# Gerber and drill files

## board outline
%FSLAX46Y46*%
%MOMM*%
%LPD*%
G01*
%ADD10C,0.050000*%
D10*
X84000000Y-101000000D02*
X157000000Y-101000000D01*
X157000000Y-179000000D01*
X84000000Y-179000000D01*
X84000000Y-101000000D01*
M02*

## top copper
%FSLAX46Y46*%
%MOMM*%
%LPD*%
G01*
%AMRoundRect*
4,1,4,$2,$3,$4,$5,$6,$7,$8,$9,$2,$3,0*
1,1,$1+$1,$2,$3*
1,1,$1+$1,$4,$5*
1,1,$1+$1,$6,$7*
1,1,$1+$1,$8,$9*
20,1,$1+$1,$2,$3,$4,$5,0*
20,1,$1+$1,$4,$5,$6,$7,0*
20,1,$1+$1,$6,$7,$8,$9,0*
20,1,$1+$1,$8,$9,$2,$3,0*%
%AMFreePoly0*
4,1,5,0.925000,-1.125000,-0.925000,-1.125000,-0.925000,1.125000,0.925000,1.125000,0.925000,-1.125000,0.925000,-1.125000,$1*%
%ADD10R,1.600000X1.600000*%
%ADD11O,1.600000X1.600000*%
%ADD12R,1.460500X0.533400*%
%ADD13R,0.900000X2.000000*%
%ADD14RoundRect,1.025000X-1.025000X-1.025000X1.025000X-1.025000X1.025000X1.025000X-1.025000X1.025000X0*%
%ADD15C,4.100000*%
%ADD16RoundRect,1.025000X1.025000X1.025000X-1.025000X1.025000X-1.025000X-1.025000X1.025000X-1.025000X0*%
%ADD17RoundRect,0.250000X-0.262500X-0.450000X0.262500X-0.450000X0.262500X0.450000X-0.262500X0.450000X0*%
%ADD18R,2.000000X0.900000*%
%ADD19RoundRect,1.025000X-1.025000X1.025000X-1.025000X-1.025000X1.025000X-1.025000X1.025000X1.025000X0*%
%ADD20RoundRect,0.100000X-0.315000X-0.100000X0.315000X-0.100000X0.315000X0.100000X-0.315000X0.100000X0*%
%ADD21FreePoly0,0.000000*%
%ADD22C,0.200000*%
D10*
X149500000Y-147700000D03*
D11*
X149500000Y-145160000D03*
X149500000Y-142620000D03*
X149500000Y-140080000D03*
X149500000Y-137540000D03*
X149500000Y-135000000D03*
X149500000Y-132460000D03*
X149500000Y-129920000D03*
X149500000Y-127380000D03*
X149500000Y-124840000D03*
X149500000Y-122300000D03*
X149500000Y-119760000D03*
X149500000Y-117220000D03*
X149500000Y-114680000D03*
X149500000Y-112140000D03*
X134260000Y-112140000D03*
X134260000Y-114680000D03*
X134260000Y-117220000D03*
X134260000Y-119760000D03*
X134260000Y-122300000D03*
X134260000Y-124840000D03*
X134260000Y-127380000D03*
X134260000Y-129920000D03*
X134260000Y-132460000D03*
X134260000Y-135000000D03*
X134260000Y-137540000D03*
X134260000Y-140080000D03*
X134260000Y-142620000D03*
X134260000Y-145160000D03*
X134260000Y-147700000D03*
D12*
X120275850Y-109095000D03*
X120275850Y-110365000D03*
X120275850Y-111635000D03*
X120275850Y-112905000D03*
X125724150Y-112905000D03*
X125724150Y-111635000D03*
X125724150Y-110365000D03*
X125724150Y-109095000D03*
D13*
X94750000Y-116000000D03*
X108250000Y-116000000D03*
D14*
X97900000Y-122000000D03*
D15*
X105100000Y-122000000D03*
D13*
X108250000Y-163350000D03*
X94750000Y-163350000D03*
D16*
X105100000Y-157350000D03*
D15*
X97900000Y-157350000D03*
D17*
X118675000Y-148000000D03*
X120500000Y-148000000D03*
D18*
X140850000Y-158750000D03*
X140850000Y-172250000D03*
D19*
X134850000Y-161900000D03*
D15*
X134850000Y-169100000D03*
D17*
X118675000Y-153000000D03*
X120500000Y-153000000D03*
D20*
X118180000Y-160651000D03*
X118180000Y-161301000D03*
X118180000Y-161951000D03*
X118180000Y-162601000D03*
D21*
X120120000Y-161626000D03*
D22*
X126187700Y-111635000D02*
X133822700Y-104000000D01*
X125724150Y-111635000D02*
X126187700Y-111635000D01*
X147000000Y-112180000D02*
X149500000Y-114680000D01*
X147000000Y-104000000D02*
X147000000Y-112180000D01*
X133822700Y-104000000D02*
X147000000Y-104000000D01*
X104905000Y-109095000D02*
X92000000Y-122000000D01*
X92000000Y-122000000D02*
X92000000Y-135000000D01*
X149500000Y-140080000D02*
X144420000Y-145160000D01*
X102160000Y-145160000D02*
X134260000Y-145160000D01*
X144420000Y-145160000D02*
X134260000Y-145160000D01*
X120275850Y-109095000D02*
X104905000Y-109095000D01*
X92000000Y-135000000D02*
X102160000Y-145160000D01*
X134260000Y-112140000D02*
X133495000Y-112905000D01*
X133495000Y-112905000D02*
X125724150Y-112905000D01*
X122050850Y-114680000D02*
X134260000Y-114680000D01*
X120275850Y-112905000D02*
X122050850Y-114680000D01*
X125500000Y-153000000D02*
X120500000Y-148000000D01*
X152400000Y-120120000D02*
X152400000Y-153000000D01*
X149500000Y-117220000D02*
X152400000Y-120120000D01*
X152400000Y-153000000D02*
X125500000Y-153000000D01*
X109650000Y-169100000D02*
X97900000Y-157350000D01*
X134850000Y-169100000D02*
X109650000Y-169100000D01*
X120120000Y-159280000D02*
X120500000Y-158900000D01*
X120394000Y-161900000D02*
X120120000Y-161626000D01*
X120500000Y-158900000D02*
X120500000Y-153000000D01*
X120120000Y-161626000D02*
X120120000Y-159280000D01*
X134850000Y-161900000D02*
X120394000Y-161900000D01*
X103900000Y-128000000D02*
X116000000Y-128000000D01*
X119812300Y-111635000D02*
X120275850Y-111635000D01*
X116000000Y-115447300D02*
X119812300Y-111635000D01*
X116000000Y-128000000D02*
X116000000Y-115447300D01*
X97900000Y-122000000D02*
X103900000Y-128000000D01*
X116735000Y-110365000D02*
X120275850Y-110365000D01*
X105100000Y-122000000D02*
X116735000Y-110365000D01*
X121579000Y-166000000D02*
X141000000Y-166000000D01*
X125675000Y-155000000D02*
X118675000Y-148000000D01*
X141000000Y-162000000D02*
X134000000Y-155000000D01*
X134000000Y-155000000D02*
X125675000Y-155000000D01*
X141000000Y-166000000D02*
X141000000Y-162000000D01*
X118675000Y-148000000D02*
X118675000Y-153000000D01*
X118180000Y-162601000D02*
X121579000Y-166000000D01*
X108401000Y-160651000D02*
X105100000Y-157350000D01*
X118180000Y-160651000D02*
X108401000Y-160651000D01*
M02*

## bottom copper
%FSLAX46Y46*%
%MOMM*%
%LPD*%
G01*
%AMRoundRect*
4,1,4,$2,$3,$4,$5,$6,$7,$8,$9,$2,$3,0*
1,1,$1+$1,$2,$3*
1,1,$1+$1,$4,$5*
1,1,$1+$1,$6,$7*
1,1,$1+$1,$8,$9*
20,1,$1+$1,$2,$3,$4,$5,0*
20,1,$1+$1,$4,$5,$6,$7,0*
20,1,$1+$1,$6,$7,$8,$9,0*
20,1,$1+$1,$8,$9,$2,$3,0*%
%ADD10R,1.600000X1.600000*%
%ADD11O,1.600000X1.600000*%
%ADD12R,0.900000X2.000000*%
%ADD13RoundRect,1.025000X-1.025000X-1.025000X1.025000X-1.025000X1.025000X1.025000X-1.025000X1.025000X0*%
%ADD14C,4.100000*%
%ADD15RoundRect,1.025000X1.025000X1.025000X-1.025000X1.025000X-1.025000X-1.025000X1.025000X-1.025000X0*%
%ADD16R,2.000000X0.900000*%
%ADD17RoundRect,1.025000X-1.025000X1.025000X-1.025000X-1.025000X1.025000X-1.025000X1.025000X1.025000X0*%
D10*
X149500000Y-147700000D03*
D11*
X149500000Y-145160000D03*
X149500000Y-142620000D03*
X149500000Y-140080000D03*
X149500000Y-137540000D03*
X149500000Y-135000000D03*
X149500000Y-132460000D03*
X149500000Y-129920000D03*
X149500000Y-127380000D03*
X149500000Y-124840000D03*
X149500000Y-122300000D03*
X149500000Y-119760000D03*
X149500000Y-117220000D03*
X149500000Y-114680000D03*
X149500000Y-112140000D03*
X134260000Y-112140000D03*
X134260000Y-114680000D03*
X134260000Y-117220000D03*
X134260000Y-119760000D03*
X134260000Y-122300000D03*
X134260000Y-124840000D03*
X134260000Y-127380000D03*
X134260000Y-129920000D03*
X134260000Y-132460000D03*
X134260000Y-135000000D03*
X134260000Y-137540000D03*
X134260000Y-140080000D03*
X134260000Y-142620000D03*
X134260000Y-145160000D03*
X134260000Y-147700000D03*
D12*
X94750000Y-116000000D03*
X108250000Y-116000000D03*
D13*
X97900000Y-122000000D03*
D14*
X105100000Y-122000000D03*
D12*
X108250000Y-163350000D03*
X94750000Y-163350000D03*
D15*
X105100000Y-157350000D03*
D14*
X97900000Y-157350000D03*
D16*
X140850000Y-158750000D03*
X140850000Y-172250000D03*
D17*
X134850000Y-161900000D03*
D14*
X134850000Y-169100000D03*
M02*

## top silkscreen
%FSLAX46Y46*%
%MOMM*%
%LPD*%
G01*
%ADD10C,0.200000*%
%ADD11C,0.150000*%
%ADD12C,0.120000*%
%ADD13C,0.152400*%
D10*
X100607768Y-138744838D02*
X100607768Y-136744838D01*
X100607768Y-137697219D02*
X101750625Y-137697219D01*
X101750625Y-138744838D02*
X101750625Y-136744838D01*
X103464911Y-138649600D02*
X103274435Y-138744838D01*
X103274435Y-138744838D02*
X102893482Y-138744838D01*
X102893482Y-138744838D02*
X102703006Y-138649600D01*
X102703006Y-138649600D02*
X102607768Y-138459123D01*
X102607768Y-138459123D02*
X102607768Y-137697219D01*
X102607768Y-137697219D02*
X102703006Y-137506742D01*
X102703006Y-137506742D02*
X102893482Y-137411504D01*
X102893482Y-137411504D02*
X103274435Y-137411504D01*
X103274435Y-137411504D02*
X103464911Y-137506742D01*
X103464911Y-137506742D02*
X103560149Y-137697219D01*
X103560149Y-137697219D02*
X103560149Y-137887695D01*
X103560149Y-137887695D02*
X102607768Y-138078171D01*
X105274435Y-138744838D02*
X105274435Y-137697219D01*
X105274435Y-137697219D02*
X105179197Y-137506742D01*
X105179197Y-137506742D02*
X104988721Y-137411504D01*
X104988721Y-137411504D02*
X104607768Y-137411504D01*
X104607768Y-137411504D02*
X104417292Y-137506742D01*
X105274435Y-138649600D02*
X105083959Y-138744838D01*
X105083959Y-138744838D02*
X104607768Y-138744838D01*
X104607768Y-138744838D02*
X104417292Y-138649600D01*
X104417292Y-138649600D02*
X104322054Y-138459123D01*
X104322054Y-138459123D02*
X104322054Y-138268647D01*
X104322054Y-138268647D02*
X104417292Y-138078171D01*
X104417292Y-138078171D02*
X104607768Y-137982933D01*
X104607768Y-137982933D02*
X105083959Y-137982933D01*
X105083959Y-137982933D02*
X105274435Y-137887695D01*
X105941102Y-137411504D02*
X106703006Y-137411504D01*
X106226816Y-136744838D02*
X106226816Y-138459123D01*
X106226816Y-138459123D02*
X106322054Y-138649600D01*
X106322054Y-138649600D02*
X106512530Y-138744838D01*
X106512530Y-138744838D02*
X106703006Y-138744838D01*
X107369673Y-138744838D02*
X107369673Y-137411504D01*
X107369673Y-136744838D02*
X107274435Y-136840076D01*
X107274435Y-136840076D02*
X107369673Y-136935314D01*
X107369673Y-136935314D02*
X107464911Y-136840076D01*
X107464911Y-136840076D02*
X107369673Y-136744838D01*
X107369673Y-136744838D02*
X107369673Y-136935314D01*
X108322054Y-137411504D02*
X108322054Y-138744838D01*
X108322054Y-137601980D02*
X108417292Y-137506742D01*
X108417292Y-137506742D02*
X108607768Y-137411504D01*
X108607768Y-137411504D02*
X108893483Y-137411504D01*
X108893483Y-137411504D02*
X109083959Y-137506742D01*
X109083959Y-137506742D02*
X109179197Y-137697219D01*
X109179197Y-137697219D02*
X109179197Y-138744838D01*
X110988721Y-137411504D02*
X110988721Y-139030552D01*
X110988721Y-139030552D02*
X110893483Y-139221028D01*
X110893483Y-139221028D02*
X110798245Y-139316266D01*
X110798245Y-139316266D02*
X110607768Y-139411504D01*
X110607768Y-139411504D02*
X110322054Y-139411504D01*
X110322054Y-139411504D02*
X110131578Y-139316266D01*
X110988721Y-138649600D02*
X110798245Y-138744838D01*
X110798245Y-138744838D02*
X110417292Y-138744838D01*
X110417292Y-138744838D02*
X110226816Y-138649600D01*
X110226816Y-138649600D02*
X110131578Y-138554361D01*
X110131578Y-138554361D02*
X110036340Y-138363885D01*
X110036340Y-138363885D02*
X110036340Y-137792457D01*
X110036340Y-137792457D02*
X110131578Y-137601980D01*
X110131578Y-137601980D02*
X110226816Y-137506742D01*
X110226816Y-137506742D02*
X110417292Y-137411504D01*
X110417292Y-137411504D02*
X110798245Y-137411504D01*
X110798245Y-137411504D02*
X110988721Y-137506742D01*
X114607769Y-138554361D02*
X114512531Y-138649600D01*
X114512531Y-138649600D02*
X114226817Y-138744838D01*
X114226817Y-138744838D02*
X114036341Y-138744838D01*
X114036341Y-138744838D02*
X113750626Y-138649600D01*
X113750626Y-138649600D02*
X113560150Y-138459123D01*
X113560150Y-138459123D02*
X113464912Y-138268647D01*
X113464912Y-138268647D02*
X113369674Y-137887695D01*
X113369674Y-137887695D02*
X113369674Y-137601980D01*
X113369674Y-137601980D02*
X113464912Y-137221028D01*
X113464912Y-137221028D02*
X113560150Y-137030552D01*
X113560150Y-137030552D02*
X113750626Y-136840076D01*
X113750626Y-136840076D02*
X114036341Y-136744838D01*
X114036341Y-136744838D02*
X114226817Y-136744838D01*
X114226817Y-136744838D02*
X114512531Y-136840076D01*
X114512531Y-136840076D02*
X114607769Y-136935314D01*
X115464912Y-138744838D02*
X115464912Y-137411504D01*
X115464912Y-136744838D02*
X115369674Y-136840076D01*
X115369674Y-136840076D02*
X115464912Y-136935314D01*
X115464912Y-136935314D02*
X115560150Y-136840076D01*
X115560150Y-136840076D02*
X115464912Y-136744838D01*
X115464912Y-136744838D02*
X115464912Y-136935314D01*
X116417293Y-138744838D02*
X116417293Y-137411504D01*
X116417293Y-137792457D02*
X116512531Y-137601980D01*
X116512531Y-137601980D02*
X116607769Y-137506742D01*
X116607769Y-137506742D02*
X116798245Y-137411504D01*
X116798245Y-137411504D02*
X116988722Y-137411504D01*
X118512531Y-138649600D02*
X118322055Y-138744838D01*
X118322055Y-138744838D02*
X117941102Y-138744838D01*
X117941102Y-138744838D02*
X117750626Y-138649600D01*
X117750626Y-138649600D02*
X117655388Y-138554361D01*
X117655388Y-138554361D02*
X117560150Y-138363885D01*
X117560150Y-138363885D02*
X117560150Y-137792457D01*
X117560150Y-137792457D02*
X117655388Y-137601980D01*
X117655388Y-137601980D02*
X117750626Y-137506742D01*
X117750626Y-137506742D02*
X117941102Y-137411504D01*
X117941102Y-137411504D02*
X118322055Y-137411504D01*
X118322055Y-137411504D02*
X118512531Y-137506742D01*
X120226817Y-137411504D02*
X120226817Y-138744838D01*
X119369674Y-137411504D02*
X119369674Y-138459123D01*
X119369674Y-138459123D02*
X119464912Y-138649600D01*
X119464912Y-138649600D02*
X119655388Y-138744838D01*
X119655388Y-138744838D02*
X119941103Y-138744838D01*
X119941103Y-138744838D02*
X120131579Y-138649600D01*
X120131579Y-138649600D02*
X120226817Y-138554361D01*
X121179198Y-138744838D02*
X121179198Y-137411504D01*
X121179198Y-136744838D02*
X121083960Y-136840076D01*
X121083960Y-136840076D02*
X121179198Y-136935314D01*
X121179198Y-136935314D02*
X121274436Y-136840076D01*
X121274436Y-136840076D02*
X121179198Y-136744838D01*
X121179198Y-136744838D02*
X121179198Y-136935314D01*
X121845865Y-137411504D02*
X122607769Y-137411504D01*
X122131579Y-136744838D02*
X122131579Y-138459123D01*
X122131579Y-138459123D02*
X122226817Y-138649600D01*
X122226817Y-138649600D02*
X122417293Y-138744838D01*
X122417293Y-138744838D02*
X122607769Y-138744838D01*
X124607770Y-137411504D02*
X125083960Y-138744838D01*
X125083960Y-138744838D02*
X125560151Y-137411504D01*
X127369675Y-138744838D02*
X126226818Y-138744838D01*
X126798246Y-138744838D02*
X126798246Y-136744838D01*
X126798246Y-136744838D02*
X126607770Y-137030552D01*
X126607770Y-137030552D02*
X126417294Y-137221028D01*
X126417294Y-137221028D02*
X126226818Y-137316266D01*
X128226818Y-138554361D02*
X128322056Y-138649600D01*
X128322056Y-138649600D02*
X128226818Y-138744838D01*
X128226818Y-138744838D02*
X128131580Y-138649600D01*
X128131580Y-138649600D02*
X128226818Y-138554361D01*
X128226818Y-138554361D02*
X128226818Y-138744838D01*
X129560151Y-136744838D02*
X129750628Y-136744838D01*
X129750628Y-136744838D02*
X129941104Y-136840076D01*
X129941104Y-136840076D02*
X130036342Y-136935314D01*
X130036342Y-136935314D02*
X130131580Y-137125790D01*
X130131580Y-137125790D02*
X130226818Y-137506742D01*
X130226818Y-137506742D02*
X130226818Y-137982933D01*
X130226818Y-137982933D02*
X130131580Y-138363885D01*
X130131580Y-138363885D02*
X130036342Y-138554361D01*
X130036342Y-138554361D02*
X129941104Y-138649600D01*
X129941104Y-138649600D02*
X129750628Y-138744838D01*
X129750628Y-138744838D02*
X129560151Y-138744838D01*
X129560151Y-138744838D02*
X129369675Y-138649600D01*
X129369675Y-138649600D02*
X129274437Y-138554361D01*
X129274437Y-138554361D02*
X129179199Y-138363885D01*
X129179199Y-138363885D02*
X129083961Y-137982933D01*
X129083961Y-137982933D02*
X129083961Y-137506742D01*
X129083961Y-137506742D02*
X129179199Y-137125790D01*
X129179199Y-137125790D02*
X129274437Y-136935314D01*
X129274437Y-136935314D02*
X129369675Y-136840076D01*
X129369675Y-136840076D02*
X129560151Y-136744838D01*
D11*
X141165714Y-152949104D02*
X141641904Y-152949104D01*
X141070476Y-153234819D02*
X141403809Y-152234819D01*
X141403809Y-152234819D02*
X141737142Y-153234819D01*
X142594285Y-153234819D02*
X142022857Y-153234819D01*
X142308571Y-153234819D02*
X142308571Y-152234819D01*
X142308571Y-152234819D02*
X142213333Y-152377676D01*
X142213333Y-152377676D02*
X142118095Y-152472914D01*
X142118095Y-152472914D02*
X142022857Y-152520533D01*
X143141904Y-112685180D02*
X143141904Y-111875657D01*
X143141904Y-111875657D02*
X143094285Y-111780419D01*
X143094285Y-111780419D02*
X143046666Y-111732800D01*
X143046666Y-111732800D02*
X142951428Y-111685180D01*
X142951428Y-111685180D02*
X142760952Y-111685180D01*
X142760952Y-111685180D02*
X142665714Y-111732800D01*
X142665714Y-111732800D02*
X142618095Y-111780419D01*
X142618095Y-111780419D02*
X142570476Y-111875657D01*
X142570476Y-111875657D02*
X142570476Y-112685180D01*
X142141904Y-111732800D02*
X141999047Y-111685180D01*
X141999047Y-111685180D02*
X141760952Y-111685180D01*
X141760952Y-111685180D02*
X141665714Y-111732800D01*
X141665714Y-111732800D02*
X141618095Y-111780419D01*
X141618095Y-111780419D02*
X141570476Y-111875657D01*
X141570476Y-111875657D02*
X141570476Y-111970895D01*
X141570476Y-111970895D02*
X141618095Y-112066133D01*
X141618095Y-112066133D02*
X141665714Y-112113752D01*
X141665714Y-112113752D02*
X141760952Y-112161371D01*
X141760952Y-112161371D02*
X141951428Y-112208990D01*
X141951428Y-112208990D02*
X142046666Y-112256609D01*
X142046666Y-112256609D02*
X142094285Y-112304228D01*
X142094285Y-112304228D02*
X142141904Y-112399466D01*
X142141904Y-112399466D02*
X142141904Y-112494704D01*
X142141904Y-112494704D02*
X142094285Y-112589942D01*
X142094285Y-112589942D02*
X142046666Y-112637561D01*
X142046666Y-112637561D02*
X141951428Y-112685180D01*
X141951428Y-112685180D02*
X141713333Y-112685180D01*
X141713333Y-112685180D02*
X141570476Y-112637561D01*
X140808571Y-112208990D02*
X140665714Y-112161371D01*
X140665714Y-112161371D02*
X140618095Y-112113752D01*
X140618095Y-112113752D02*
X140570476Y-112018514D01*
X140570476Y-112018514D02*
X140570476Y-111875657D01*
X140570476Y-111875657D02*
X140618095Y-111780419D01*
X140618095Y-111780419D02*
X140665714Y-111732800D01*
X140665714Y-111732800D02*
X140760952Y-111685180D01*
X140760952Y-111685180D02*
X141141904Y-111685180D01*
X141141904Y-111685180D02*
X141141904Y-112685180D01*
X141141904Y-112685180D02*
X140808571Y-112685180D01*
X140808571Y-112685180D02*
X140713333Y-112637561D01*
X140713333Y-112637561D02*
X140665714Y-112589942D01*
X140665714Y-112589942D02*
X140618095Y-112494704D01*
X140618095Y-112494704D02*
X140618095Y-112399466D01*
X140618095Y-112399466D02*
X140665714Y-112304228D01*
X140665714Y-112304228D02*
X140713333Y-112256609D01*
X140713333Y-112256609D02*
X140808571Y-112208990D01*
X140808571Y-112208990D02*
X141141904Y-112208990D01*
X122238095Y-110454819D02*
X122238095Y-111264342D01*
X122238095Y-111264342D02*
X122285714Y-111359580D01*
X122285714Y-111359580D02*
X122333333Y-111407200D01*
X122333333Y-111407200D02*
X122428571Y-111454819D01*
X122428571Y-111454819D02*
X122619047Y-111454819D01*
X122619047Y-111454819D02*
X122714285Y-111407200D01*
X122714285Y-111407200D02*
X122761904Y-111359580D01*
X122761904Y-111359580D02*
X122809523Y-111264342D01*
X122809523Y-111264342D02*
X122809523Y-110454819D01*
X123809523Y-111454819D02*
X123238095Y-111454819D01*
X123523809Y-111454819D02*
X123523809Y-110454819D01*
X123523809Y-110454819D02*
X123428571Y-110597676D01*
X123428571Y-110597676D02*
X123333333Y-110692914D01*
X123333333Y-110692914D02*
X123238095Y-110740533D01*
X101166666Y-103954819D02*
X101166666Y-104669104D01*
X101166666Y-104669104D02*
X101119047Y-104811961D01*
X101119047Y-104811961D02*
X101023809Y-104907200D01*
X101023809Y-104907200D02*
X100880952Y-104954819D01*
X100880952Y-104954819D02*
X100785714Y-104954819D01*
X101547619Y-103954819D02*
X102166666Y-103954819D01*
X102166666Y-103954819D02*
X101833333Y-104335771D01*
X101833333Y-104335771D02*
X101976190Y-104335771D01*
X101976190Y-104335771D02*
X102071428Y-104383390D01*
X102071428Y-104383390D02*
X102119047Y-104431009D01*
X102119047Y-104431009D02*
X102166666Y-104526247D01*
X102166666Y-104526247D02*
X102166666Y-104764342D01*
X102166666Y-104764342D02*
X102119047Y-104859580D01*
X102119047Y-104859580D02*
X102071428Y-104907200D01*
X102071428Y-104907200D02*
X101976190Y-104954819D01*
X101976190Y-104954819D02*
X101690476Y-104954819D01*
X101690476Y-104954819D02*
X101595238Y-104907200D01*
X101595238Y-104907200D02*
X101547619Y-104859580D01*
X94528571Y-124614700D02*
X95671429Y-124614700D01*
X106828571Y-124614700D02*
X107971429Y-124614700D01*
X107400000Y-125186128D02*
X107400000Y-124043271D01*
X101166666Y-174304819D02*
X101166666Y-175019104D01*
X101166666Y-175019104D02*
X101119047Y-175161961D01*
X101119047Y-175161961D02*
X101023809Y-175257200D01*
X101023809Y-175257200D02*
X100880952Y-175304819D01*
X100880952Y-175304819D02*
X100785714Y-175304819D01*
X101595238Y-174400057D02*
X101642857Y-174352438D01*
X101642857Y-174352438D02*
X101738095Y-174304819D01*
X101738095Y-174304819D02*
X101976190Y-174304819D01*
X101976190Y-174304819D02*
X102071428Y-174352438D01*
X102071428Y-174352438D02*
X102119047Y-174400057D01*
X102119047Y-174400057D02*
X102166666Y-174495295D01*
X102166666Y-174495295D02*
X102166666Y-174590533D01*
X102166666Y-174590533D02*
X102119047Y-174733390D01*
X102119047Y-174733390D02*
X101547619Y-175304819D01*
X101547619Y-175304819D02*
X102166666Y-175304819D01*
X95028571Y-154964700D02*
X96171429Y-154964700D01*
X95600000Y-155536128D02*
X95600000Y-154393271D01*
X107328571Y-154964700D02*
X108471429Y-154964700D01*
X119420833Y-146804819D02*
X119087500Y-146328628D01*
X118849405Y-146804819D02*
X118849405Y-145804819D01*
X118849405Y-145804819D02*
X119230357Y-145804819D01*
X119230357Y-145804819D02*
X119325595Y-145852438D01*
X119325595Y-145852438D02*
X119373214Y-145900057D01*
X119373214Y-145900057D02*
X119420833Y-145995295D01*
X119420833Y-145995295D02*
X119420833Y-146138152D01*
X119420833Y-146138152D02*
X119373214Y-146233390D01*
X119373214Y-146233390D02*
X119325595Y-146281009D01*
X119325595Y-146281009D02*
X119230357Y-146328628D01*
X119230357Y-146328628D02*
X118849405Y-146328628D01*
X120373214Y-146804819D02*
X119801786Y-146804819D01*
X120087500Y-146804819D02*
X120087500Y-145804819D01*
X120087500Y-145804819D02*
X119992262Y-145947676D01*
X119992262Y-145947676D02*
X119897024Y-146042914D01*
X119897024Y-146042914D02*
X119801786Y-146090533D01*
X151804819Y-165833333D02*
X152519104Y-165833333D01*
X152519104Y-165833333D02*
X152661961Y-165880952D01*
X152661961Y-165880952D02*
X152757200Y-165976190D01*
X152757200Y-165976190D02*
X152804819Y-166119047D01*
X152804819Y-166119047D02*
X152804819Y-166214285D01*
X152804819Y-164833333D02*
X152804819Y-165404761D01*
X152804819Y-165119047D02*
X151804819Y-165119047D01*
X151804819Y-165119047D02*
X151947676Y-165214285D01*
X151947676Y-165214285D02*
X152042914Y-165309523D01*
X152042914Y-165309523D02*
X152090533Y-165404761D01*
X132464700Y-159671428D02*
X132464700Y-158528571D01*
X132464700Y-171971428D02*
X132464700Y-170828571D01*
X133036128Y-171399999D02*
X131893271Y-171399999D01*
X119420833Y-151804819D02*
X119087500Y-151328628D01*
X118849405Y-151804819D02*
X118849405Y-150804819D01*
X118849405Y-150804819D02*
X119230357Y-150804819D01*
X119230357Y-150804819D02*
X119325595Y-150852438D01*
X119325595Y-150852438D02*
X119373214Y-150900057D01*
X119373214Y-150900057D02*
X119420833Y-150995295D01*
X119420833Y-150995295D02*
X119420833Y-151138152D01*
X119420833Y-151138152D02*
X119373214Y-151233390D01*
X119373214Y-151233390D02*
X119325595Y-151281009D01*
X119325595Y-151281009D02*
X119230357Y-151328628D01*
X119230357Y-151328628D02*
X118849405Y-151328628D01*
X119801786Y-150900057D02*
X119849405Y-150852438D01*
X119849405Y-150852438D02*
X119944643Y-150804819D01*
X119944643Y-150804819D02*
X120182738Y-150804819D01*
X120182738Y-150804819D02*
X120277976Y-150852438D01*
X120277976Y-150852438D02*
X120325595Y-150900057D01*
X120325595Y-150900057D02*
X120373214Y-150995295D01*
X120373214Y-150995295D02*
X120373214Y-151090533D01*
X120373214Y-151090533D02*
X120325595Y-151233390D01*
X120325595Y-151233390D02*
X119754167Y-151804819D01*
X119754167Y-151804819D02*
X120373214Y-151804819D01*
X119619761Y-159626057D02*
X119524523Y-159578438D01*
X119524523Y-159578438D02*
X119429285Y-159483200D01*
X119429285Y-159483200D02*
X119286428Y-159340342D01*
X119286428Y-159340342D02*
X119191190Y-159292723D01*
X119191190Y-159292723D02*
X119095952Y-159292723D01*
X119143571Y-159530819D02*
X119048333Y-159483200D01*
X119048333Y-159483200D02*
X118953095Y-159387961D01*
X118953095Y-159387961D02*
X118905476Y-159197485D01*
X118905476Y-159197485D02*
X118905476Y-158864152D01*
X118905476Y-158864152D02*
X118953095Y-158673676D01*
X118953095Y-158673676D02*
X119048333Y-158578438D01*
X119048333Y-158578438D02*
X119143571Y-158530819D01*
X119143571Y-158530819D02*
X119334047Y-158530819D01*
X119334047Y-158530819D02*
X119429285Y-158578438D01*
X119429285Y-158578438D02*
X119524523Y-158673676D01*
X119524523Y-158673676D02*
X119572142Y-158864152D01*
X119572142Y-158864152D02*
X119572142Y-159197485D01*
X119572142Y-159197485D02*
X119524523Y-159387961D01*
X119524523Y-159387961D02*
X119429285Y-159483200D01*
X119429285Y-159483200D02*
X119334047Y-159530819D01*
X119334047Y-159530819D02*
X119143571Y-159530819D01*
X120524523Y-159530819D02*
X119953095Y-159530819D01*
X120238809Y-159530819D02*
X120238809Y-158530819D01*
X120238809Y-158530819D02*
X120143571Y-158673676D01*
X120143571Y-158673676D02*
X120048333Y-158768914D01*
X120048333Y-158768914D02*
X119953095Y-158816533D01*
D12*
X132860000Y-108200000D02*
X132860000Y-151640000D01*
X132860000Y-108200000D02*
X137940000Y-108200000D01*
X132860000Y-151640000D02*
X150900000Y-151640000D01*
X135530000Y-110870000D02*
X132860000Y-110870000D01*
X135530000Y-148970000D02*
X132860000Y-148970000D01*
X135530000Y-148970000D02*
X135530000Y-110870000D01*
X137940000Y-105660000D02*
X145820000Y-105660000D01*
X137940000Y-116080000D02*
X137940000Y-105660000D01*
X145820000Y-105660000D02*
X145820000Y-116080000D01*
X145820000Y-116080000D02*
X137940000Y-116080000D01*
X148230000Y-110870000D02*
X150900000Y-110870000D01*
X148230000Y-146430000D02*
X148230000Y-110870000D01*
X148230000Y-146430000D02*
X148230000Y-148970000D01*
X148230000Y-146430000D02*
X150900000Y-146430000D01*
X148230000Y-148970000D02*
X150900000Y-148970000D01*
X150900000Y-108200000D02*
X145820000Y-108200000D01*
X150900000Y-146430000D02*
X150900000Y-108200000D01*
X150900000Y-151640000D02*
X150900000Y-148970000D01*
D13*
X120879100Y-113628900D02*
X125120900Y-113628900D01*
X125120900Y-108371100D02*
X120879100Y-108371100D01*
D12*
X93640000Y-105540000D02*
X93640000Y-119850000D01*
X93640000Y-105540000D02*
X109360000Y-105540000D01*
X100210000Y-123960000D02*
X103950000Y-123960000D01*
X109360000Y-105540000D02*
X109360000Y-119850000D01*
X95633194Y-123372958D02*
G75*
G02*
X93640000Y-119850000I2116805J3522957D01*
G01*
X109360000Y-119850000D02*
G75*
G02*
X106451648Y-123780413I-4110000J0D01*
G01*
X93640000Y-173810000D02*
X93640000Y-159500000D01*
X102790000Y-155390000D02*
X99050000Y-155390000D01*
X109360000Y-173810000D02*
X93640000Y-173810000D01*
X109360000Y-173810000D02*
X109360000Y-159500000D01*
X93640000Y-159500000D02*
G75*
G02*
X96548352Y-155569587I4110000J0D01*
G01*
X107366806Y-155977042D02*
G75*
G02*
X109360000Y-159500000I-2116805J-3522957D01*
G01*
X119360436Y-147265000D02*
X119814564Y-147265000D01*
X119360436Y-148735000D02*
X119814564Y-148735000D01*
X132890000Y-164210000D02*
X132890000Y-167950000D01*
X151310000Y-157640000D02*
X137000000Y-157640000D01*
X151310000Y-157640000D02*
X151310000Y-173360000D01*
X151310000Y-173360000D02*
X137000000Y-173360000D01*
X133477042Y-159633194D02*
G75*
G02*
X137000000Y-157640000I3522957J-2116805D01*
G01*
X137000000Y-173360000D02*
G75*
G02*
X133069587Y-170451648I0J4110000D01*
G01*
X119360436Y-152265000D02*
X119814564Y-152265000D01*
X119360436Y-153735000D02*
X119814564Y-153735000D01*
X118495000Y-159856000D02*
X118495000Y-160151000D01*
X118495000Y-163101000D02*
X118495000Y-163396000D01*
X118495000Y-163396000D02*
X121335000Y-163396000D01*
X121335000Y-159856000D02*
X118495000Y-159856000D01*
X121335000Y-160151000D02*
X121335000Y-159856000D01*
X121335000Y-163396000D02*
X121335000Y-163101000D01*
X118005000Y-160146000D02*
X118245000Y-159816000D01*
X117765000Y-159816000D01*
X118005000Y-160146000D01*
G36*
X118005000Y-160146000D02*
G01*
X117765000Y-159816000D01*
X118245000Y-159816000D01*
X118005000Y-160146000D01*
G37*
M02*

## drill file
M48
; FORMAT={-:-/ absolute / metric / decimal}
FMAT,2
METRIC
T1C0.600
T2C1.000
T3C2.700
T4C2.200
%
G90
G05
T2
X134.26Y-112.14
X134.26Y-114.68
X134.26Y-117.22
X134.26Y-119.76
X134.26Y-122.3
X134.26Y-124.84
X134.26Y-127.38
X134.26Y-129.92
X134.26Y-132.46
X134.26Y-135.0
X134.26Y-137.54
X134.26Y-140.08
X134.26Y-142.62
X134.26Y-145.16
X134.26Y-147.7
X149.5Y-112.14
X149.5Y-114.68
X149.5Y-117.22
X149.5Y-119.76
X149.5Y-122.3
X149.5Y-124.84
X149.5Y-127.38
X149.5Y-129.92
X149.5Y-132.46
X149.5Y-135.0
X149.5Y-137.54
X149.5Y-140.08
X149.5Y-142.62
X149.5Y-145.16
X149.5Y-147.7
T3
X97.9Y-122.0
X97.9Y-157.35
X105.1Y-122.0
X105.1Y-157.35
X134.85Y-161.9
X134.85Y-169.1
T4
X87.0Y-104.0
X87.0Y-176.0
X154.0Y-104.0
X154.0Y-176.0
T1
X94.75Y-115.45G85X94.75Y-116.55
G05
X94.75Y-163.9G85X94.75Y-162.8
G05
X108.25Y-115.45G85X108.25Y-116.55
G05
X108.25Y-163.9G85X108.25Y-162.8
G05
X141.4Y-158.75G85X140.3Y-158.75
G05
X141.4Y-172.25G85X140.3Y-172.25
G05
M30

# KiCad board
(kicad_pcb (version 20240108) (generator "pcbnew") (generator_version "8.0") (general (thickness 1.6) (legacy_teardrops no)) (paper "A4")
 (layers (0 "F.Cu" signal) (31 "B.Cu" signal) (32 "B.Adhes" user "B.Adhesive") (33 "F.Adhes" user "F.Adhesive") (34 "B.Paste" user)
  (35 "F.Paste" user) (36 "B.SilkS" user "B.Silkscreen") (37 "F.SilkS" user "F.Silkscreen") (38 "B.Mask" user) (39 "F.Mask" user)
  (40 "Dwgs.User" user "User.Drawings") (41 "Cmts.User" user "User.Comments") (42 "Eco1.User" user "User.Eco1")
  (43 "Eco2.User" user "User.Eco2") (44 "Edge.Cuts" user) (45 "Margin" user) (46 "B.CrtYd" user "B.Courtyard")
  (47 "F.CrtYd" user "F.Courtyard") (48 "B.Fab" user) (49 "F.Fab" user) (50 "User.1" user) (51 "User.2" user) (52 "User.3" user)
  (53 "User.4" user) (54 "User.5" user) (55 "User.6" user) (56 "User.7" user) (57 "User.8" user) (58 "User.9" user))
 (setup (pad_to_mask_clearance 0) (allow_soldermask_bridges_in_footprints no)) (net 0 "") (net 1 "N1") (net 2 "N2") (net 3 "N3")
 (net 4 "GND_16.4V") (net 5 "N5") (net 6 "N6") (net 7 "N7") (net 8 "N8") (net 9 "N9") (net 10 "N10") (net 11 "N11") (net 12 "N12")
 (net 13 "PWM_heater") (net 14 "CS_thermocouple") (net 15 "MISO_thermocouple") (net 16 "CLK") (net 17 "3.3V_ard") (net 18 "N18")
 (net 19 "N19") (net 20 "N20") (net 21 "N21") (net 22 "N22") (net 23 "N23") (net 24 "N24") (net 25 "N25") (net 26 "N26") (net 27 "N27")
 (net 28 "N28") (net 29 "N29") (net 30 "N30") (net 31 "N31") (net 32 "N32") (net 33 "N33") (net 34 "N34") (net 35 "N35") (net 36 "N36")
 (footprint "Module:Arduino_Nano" (layer "F.Cu") (at 149.5 147.7 180)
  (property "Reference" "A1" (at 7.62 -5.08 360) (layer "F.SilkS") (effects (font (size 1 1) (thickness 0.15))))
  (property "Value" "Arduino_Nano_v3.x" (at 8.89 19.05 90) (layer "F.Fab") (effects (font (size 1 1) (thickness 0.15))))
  (fp_line (start 16.64 39.5) (end 16.64 -3.94) (stroke (width 0.12) (type solid)) (layer "F.SilkS"))
  (fp_line (start 16.64 39.5) (end 11.56 39.5) (stroke (width 0.12) (type solid)) (layer "F.SilkS"))
  (fp_line (start 16.64 -3.94) (end -1.4 -3.94) (stroke (width 0.12) (type solid)) (layer "F.SilkS"))
  (fp_line (start 13.97 36.83) (end 16.64 36.83) (stroke (width 0.12) (type solid)) (layer "F.SilkS"))
  (fp_line (start 13.97 -1.27) (end 16.64 -1.27) (stroke (width 0.12) (type solid)) (layer "F.SilkS"))
  (fp_line (start 13.97 -1.27) (end 13.97 36.83) (stroke (width 0.12) (type solid)) (layer "F.SilkS"))
  (fp_line (start 11.56 42.04) (end 3.68 42.04) (stroke (width 0.12) (type solid)) (layer "F.SilkS"))
  (fp_line (start 11.56 31.62) (end 11.56 42.04) (stroke (width 0.12) (type solid)) (layer "F.SilkS"))
  (fp_line (start 3.68 42.04) (end 3.68 31.62) (stroke (width 0.12) (type solid)) (layer "F.SilkS"))
  (fp_line (start 3.68 31.62) (end 11.56 31.62) (stroke (width 0.12) (type solid)) (layer "F.SilkS"))
  (fp_line (start 1.27 36.83) (end -1.4 36.83) (stroke (width 0.12) (type solid)) (layer "F.SilkS"))
  (fp_line (start 1.27 1.27) (end 1.27 36.83) (stroke (width 0.12) (type solid)) (layer "F.SilkS"))
  (fp_line (start 1.27 1.27) (end 1.27 -1.27) (stroke (width 0.12) (type solid)) (layer "F.SilkS"))
  (fp_line (start 1.27 1.27) (end -1.4 1.27) (stroke (width 0.12) (type solid)) (layer "F.SilkS"))
  (fp_line (start 1.27 -1.27) (end -1.4 -1.27) (stroke (width 0.12) (type solid)) (layer "F.SilkS"))
  (fp_line (start -1.4 39.5) (end 3.68 39.5) (stroke (width 0.12) (type solid)) (layer "F.SilkS"))
  (fp_line (start -1.4 1.27) (end -1.4 39.5) (stroke (width 0.12) (type solid)) (layer "F.SilkS"))
  (fp_line (start -1.4 -3.94) (end -1.4 -1.27) (stroke (width 0.12) (type solid)) (layer "F.SilkS"))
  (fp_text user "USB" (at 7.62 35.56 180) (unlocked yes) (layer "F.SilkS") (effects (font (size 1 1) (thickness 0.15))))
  (pad "1" thru_hole rect (at 0 0 180) (size 1.6 1.6) (drill 1) (layers "*.Cu" "*.Mask") (remove_unused_layers no) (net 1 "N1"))
  (pad "2" thru_hole oval (at 0 2.54 180) (size 1.6 1.6) (drill 1) (layers "*.Cu" "*.Mask") (remove_unused_layers no) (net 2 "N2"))
  (pad "3" thru_hole oval (at 0 5.08 180) (size 1.6 1.6) (drill 1) (layers "*.Cu" "*.Mask") (remove_unused_layers no) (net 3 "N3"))
  (pad "4" thru_hole oval (at 0 7.62 180) (size 1.6 1.6) (drill 1) (layers "*.Cu" "*.Mask") (remove_unused_layers no) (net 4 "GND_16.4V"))
  (pad "5" thru_hole oval (at 0 10.16 180) (size 1.6 1.6) (drill 1) (layers "*.Cu" "*.Mask") (remove_unused_layers no) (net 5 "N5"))
  (pad "6" thru_hole oval (at 0 12.7 180) (size 1.6 1.6) (drill 1) (layers "*.Cu" "*.Mask") (remove_unused_layers no) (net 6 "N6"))
  (pad "7" thru_hole oval (at 0 15.24 180) (size 1.6 1.6) (drill 1) (layers "*.Cu" "*.Mask") (remove_unused_layers no) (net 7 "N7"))
  (pad "8" thru_hole oval (at 0 17.78 180) (size 1.6 1.6) (drill 1) (layers "*.Cu" "*.Mask") (remove_unused_layers no) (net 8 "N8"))
  (pad "9" thru_hole oval (at 0 20.32 180) (size 1.6 1.6) (drill 1) (layers "*.Cu" "*.Mask") (remove_unused_layers no) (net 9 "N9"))
  (pad "10" thru_hole oval (at 0 22.86 180) (size 1.6 1.6) (drill 1) (layers "*.Cu" "*.Mask") (remove_unused_layers no) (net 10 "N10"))
  (pad "11" thru_hole oval (at 0 25.4 180) (size 1.6 1.6) (drill 1) (layers "*.Cu" "*.Mask") (remove_unused_layers no) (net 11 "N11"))
  (pad "12" thru_hole oval (at 0 27.94 180) (size 1.6 1.6) (drill 1) (layers "*.Cu" "*.Mask") (remove_unused_layers no) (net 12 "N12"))
  (pad "13" thru_hole oval (at 0 30.48 180) (size 1.6 1.6) (drill 1) (layers "*.Cu" "*.Mask") (remove_unused_layers no)
   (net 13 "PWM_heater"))
  (pad "14" thru_hole oval (at 0 33.02 180) (size 1.6 1.6) (drill 1) (layers "*.Cu" "*.Mask") (remove_unused_layers no)
   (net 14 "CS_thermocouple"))
  (pad "15" thru_hole oval (at 0 35.56 180) (size 1.6 1.6) (drill 1) (layers "*.Cu" "*.Mask") (remove_unused_layers no)
   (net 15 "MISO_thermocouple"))
  (pad "16" thru_hole oval (at 15.24 35.56 180) (size 1.6 1.6) (drill 1) (layers "*.Cu" "*.Mask") (remove_unused_layers no) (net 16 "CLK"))
  (pad "17" thru_hole oval (at 15.24 33.02 180) (size 1.6 1.6) (drill 1) (layers "*.Cu" "*.Mask") (remove_unused_layers no)
   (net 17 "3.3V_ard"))
  (pad "18" thru_hole oval (at 15.24 30.48 180) (size 1.6 1.6) (drill 1) (layers "*.Cu" "*.Mask") (remove_unused_layers no) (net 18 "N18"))
  (pad "19" thru_hole oval (at 15.24 27.94 180) (size 1.6 1.6) (drill 1) (layers "*.Cu" "*.Mask") (remove_unused_layers no) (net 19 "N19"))
  (pad "20" thru_hole oval (at 15.24 25.4 180) (size 1.6 1.6) (drill 1) (layers "*.Cu" "*.Mask") (remove_unused_layers no) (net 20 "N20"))
  (pad "21" thru_hole oval (at 15.24 22.86 180) (size 1.6 1.6) (drill 1) (layers "*.Cu" "*.Mask") (remove_unused_layers no) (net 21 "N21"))
  (pad "22" thru_hole oval (at 15.24 20.32 180) (size 1.6 1.6) (drill 1) (layers "*.Cu" "*.Mask") (remove_unused_layers no) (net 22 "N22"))
  (pad "23" thru_hole oval (at 15.24 17.78 180) (size 1.6 1.6) (drill 1) (layers "*.Cu" "*.Mask") (remove_unused_layers no) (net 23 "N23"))
  (pad "24" thru_hole oval (at 15.24 15.24 180) (size 1.6 1.6) (drill 1) (layers "*.Cu" "*.Mask") (remove_unused_layers no) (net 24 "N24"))
  (pad "25" thru_hole oval (at 15.24 12.7 180) (size 1.6 1.6) (drill 1) (layers "*.Cu" "*.Mask") (remove_unused_layers no) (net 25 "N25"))
  (pad "26" thru_hole oval (at 15.24 10.16 180) (size 1.6 1.6) (drill 1) (layers "*.Cu" "*.Mask") (remove_unused_layers no) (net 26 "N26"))
  (pad "27" thru_hole oval (at 15.24 7.62 180) (size 1.6 1.6) (drill 1) (layers "*.Cu" "*.Mask") (remove_unused_layers no) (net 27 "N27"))
  (pad "28" thru_hole oval (at 15.24 5.08 180) (size 1.6 1.6) (drill 1) (layers "*.Cu" "*.Mask") (remove_unused_layers no) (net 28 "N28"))
  (pad "29" thru_hole oval (at 15.24 2.54 180) (size 1.6 1.6) (drill 1) (layers "*.Cu" "*.Mask") (remove_unused_layers no)
   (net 4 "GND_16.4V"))
  (pad "30" thru_hole oval (at 15.24 0 180) (size 1.6 1.6) (drill 1) (layers "*.Cu" "*.Mask") (remove_unused_layers no) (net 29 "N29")))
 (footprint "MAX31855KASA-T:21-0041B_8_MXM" (layer "F.Cu") (at 123 111)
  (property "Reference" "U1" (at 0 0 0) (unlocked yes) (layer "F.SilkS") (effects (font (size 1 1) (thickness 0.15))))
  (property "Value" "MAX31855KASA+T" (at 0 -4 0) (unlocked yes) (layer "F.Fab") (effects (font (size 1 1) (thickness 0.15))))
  (fp_line (start -2.1209 2.6289) (end 2.1209 2.6289) (stroke (width 0.1524) (type solid)) (layer "F.SilkS"))
  (fp_line (start 2.1209 -2.6289) (end -2.1209 -2.6289) (stroke (width 0.1524) (type solid)) (layer "F.SilkS"))
  (pad "1" smd rect (at -2.72415 -1.905) (size 1.4605 0.5334) (layers "F.Cu" "F.Paste" "F.Mask") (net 4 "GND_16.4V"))
  (pad "2" smd rect (at -2.72415 -0.635) (size 1.4605 0.5334) (layers "F.Cu" "F.Paste" "F.Mask") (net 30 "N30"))
  (pad "3" smd rect (at -2.72415 0.635) (size 1.4605 0.5334) (layers "F.Cu" "F.Paste" "F.Mask") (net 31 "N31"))
  (pad "4" smd rect (at -2.72415 1.905) (size 1.4605 0.5334) (layers "F.Cu" "F.Paste" "F.Mask") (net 17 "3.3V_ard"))
  (pad "5" smd rect (at 2.72415 1.905) (size 1.4605 0.5334) (layers "F.Cu" "F.Paste" "F.Mask") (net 16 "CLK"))
  (pad "6" smd rect (at 2.72415 0.635) (size 1.4605 0.5334) (layers "F.Cu" "F.Paste" "F.Mask") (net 14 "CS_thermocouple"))
  (pad "7" smd rect (at 2.72415 -0.635) (size 1.4605 0.5334) (layers "F.Cu" "F.Paste" "F.Mask") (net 15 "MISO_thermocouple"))
  (pad "8" smd rect (at 2.72415 -1.905) (size 1.4605 0.5334) (layers "F.Cu" "F.Paste" "F.Mask") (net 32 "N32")))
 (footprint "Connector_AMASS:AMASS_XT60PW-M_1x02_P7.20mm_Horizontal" (layer "F.Cu") (at 97.9 122)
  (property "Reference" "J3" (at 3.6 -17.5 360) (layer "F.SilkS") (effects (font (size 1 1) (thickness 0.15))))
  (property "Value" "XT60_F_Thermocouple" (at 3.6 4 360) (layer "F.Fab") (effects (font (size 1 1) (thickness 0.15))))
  (fp_line (start -4.26 -16.46) (end -4.26 -2.15) (stroke (width 0.12) (type solid)) (layer "F.SilkS"))
  (fp_line (start -4.26 -16.46) (end 11.46 -16.46) (stroke (width 0.12) (type solid)) (layer "F.SilkS"))
  (fp_line (start 2.31 1.96) (end 6.05 1.96) (stroke (width 0.12) (type solid)) (layer "F.SilkS"))
  (fp_line (start 11.46 -16.46) (end 11.46 -2.15) (stroke (width 0.12) (type solid)) (layer "F.SilkS"))
  (fp_arc (start -2.266806 1.372958) (mid -3.727162 -0.126139) (end -4.26 -2.15) (stroke (width 0.12) (type solid)) (layer "F.SilkS"))
  (fp_arc (start 11.46 -2.15) (mid 10.653852 0.294722) (end 8.551648 1.780413) (stroke (width 0.12) (type solid)) (layer "F.SilkS"))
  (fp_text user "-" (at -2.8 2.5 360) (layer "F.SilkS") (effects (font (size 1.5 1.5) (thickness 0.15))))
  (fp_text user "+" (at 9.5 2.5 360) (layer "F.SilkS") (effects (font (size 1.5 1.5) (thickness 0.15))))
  (pad "" thru_hole rect (at -3.15 -6) (size 0.9 2) (drill oval 0.6 1.7) (layers "*.Cu" "*.Mask") (remove_unused_layers no))
  (pad "" thru_hole rect (at 10.35 -6) (size 0.9 2) (drill oval 0.6 1.7) (layers "*.Cu" "*.Mask") (remove_unused_layers no))
  (pad "1" thru_hole roundrect (at 0 0) (size 4.1 4.1) (drill 2.7) (layers "*.Cu" "*.Mask") (remove_unused_layers no)
   (roundrect_rratio 0.25) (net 31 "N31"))
  (pad "2" thru_hole circle (at 7.2 0) (size 4.1 4.1) (drill 2.7) (layers "*.Cu" "*.Mask") (remove_unused_layers no) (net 30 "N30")))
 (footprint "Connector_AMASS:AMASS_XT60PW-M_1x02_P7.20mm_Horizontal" (layer "F.Cu") (at 105.1 157.35 180)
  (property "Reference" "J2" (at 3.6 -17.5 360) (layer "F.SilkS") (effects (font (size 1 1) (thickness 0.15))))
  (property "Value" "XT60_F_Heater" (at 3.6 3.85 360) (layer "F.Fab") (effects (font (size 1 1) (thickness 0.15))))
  (fp_line (start 11.46 -16.46) (end 11.46 -2.15) (stroke (width 0.12) (type solid)) (layer "F.SilkS"))
  (fp_line (start 2.31 1.96) (end 6.05 1.96) (stroke (width 0.12) (type solid)) (layer "F.SilkS"))
  (fp_line (start -4.26 -16.46) (end 11.46 -16.46) (stroke (width 0.12) (type solid)) (layer "F.SilkS"))
  (fp_line (start -4.26 -16.46) (end -4.26 -2.15) (stroke (width 0.12) (type solid)) (layer "F.SilkS"))
  (fp_arc (start 11.46 -2.15) (mid 10.653852 0.294722) (end 8.551648 1.780413) (stroke (width 0.12) (type solid)) (layer "F.SilkS"))
  (fp_arc (start -2.266806 1.372958) (mid -3.727162 -0.126139) (end -4.26 -2.15) (stroke (width 0.12) (type solid)) (layer "F.SilkS"))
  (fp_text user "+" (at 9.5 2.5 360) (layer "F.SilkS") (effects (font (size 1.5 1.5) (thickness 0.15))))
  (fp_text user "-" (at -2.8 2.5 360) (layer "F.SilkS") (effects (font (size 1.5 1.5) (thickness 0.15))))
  (pad "" thru_hole rect (at -3.15 -6 180) (size 0.9 2) (drill oval 0.6 1.7) (layers "*.Cu" "*.Mask") (remove_unused_layers no))
  (pad "" thru_hole rect (at 10.35 -6 180) (size 0.9 2) (drill oval 0.6 1.7) (layers "*.Cu" "*.Mask") (remove_unused_layers no))
  (pad "1" thru_hole roundrect (at 0 0 180) (size 4.1 4.1) (drill 2.7) (layers "*.Cu" "*.Mask") (remove_unused_layers no)
   (roundrect_rratio 0.25) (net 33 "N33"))
  (pad "2" thru_hole circle (at 7.2 0 180) (size 4.1 4.1) (drill 2.7) (layers "*.Cu" "*.Mask") (remove_unused_layers no) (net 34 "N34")))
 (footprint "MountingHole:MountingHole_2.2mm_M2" (layer "F.Cu") (at 154 104)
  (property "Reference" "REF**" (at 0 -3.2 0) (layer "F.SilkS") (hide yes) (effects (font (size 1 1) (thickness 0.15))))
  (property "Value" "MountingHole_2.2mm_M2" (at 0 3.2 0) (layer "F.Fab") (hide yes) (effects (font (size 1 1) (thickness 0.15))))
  (pad "" np_thru_hole circle (at 0 0) (size 2.2 2.2) (drill 2.2) (layers "*.Cu" "*.Mask")))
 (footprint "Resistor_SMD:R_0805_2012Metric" (layer "F.Cu") (at 119.5875 148)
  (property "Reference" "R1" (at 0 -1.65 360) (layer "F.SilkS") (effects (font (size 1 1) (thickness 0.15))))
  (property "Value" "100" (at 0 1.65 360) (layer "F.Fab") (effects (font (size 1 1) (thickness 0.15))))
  (fp_line (start -0.227064 -0.735) (end 0.227064 -0.735) (stroke (width 0.12) (type solid)) (layer "F.SilkS"))
  (fp_line (start -0.227064 0.735) (end 0.227064 0.735) (stroke (width 0.12) (type solid)) (layer "F.SilkS"))
  (pad "1" smd roundrect (at -0.9125 0) (size 1.025 1.4) (layers "F.Cu" "F.Paste" "F.Mask") (roundrect_rratio 0.243902) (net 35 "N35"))
  (pad "2" smd roundrect (at 0.9125 0) (size 1.025 1.4) (layers "F.Cu" "F.Paste" "F.Mask") (roundrect_rratio 0.243902) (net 13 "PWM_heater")))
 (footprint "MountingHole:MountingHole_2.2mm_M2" (layer "F.Cu") (at 154 176)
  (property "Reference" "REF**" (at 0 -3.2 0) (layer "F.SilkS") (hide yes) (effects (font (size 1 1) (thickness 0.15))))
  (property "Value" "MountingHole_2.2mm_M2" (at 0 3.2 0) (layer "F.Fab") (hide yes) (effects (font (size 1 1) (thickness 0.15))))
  (pad "" np_thru_hole circle (at 0 0) (size 2.2 2.2) (drill 2.2) (layers "*.Cu" "*.Mask")))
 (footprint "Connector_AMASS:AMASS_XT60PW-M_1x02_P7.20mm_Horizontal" (layer "F.Cu") (at 134.85 161.9 -90)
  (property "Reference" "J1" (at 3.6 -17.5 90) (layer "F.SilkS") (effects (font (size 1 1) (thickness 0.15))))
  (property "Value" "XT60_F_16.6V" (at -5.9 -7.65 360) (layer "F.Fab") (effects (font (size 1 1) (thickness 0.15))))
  (fp_line (start 2.31 1.96) (end 6.05 1.96) (stroke (width 0.12) (type solid)) (layer "F.SilkS"))
  (fp_line (start -4.26 -16.46) (end -4.26 -2.15) (stroke (width 0.12) (type solid)) (layer "F.SilkS"))
  (fp_line (start -4.26 -16.46) (end 11.46 -16.46) (stroke (width 0.12) (type solid)) (layer "F.SilkS"))
  (fp_line (start 11.46 -16.46) (end 11.46 -2.15) (stroke (width 0.12) (type solid)) (layer "F.SilkS"))
  (fp_arc (start -2.266806 1.372958) (mid -3.727162 -0.126139) (end -4.26 -2.15) (stroke (width 0.12) (type solid)) (layer "F.SilkS"))
  (fp_arc (start 11.46 -2.15) (mid 10.653852 0.294722) (end 8.551648 1.780413) (stroke (width 0.12) (type solid)) (layer "F.SilkS"))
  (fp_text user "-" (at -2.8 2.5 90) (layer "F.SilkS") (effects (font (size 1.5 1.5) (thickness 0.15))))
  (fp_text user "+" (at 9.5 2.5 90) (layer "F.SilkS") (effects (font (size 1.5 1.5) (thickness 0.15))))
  (pad "" thru_hole rect (at -3.15 -6 270) (size 0.9 2) (drill oval 0.6 1.7) (layers "*.Cu" "*.Mask") (remove_unused_layers no))
  (pad "" thru_hole rect (at 10.35 -6 270) (size 0.9 2) (drill oval 0.6 1.7) (layers "*.Cu" "*.Mask") (remove_unused_layers no))
  (pad "1" thru_hole roundrect (at 0 0 270) (size 4.1 4.1) (drill 2.7) (layers "*.Cu" "*.Mask") (remove_unused_layers no)
   (roundrect_rratio 0.25) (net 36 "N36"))
  (pad "2" thru_hole circle (at 7.2 0 270) (size 4.1 4.1) (drill 2.7) (layers "*.Cu" "*.Mask") (remove_unused_layers no) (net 34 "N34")))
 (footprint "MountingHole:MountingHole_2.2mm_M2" (layer "F.Cu") (at 87 176)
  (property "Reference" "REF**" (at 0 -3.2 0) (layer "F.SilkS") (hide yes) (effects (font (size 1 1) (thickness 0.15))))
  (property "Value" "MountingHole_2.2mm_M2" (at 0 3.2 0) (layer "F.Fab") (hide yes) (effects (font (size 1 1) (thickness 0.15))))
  (pad "" np_thru_hole circle (at 0 0) (size 2.2 2.2) (drill 2.2) (layers "*.Cu" "*.Mask")))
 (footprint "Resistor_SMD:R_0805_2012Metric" (layer "F.Cu") (at 119.5875 153)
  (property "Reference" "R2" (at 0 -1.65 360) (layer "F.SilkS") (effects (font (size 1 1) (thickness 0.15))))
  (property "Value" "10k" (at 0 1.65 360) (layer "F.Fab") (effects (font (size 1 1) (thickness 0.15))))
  (fp_line (start -0.227064 -0.735) (end 0.227064 -0.735) (stroke (width 0.12) (type solid)) (layer "F.SilkS"))
  (fp_line (start -0.227064 0.735) (end 0.227064 0.735) (stroke (width 0.12) (type solid)) (layer "F.SilkS"))
  (pad "1" smd roundrect (at -0.9125 0) (size 1.025 1.4) (layers "F.Cu" "F.Paste" "F.Mask") (roundrect_rratio 0.243902) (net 35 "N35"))
  (pad "2" smd roundrect (at 0.9125 0) (size 1.025 1.4) (layers "F.Cu" "F.Paste" "F.Mask") (roundrect_rratio 0.243902) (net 36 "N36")))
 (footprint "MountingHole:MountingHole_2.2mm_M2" (layer "F.Cu") (at 87 104)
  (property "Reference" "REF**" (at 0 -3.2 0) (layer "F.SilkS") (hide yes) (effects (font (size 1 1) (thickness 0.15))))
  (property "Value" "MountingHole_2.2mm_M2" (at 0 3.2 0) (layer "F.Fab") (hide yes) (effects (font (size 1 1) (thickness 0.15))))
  (pad "" np_thru_hole circle (at 0 0) (size 2.2 2.2) (drill 2.2) (layers "*.Cu" "*.Mask")))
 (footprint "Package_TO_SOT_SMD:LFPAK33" (layer "F.Cu") (at 119.715 161.626)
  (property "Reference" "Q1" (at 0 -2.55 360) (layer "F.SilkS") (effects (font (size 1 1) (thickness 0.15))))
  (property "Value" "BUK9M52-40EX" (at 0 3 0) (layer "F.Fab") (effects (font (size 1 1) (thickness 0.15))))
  (fp_line (start -1.22 -1.77) (end -1.22 -1.475) (stroke (width 0.12) (type solid)) (layer "F.SilkS"))
  (fp_line (start -1.22 1.475) (end -1.22 1.77) (stroke (width 0.12) (type solid)) (layer "F.SilkS"))
  (fp_line (start -1.22 1.77) (end 1.62 1.77) (stroke (width 0.12) (type solid)) (layer "F.SilkS"))
  (fp_line (start 1.62 -1.77) (end -1.22 -1.77) (stroke (width 0.12) (type solid)) (layer "F.SilkS"))
  (fp_line (start 1.62 -1.475) (end 1.62 -1.77) (stroke (width 0.12) (type solid)) (layer "F.SilkS"))
  (fp_line (start 1.62 1.77) (end 1.62 1.475) (stroke (width 0.12) (type solid)) (layer "F.SilkS"))
  (fp_poly
   (pts (xy -1.71 -1.48) (xy -1.47 -1.81) (xy -1.95 -1.81) (xy -1.71 -1.48)) (stroke (width 0.12) (type solid)) (fill solid)
   (layer "F.SilkS"))
  (pad "" smd roundrect (at -1.535 -0.975) (size 0.83 0.3) (layers "F.Paste") (roundrect_rratio 0.25))
  (pad "" smd roundrect (at -1.535 -0.325) (size 0.83 0.3) (layers "F.Paste") (roundrect_rratio 0.25))
  (pad "" smd roundrect (at -1.535 0.325) (size 0.83 0.3) (layers "F.Paste") (roundrect_rratio 0.25))
  (pad "" smd roundrect (at -1.535 0.975) (size 0.83 0.3) (layers "F.Paste") (roundrect_rratio 0.25))
  (pad "" smd roundrect (at -0.215 -0.626) (size 0.51 0.635) (layers "F.Paste") (roundrect_rratio 0.25))
  (pad "" smd roundrect (at -0.215 0.626) (size 0.51 0.635) (layers "F.Paste") (roundrect_rratio 0.25))
  (pad "" smd roundrect (at 0.645 -0.626) (size 0.51 0.635) (layers "F.Paste") (roundrect_rratio 0.25))
  (pad "" smd roundrect (at 0.645 0.626) (size 0.51 0.635) (layers "F.Paste") (roundrect_rratio 0.25))
  (pad "" smd roundrect (at 1.575 -0.975) (size 0.83 0.3) (layers "F.Paste") (roundrect_rratio 0.25))
  (pad "" smd roundrect (at 1.575 -0.325) (size 0.83 0.3) (layers "F.Paste") (roundrect_rratio 0.25))
  (pad "" smd roundrect (at 1.575 0.325) (size 0.83 0.3) (layers "F.Paste") (roundrect_rratio 0.25))
  (pad "" smd roundrect (at 1.575 0.975) (size 0.83 0.3) (layers "F.Paste") (roundrect_rratio 0.25))
  (pad "1" smd roundrect (at -1.535 -0.975) (size 0.83 0.4) (layers "F.Cu" "F.Mask") (roundrect_rratio 0.25) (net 33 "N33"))
  (pad "2" smd roundrect (at -1.535 -0.325) (size 0.83 0.4) (layers "F.Cu" "F.Mask") (roundrect_rratio 0.25) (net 33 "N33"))
  (pad "3" smd roundrect (at -1.535 0.325) (size 0.83 0.4) (layers "F.Cu" "F.Mask") (roundrect_rratio 0.25) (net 33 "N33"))
  (pad "4" smd roundrect (at -1.535 0.975) (size 0.83 0.4) (layers "F.Cu" "F.Mask") (roundrect_rratio 0.25) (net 35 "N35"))
  (pad "5" smd custom (at 0.405 0) (size 1.85 2.25) (layers "F.Cu" "F.Mask") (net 36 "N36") (zone_connect 2) (thermal_bridge_angle 45)
   (options (clearance outline) (anchor rect)) (primitives)))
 (gr_rect (start 84 101) (end 157 179) (stroke (width 0.05) (type default)) (fill none) (layer "Edge.Cuts"))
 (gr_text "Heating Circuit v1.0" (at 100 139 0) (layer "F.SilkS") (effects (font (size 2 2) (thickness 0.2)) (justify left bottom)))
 (segment (start 126.1877 111.635) (end 133.8227 104) (width 0.2) (layer "F.Cu") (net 14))
 (segment (start 125.72415 111.635) (end 126.1877 111.635) (width 0.2) (layer "F.Cu") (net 14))
 (segment (start 147 112.18) (end 149.5 114.68) (width 0.2) (layer "F.Cu") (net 14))
 (segment (start 147 104) (end 147 112.18) (width 0.2) (layer "F.Cu") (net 14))
 (segment (start 133.8227 104) (end 147 104) (width 0.2) (layer "F.Cu") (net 14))
 (segment (start 104.905 109.095) (end 92 122) (width 0.2) (layer "F.Cu") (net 4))
 (segment (start 92 122) (end 92 135) (width 0.2) (layer "F.Cu") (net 4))
 (segment (start 149.5 140.08) (end 144.42 145.16) (width 0.2) (layer "F.Cu") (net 4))
 (segment (start 102.16 145.16) (end 134.26 145.16) (width 0.2) (layer "F.Cu") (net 4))
 (segment (start 144.42 145.16) (end 134.26 145.16) (width 0.2) (layer "F.Cu") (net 4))
 (segment (start 120.27585 109.095) (end 104.905 109.095) (width 0.2) (layer "F.Cu") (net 4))
 (segment (start 92 135) (end 102.16 145.16) (width 0.2) (layer "F.Cu") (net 4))
 (segment (start 134.26 112.14) (end 133.495 112.905) (width 0.2) (layer "F.Cu") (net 16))
 (segment (start 133.495 112.905) (end 125.72415 112.905) (width 0.2) (layer "F.Cu") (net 16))
 (segment (start 122.05085 114.68) (end 134.26 114.68) (width 0.2) (layer "F.Cu") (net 17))
 (segment (start 120.27585 112.905) (end 122.05085 114.68) (width 0.2) (layer "F.Cu") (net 17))
 (segment (start 125.5 153) (end 120.5 148) (width 0.2) (layer "F.Cu") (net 13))
 (segment (start 152.4 120.12) (end 152.4 153) (width 0.2) (layer "F.Cu") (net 13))
 (segment (start 149.5 117.22) (end 152.4 120.12) (width 0.2) (layer "F.Cu") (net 13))
 (segment (start 152.4 153) (end 125.5 153) (width 0.2) (layer "F.Cu") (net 13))
 (segment (start 109.65 169.1) (end 97.9 157.35) (width 0.2) (layer "F.Cu") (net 34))
 (segment (start 134.85 169.1) (end 109.65 169.1) (width 0.2) (layer "F.Cu") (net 34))
 (segment (start 120.12 159.28) (end 120.5 158.9) (width 0.2) (layer "F.Cu") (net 36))
 (segment (start 120.394 161.9) (end 120.12 161.626) (width 0.2) (layer "F.Cu") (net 36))
 (segment (start 120.5 158.9) (end 120.5 153) (width 0.2) (layer "F.Cu") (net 36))
 (segment (start 120.12 161.626) (end 120.12 159.28) (width 0.2) (layer "F.Cu") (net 36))
 (segment (start 134.85 161.9) (end 120.394 161.9) (width 0.2) (layer "F.Cu") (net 36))
 (segment (start 103.9 128) (end 116 128) (width 0.2) (layer "F.Cu") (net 31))
 (segment (start 119.8123 111.635) (end 120.27585 111.635) (width 0.2) (layer "F.Cu") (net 31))
 (segment (start 116 115.4473) (end 119.8123 111.635) (width 0.2) (layer "F.Cu") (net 31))
 (segment (start 116 128) (end 116 115.4473) (width 0.2) (layer "F.Cu") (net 31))
 (segment (start 97.9 122) (end 103.9 128) (width 0.2) (layer "F.Cu") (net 31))
 (segment (start 116.735 110.365) (end 120.27585 110.365) (width 0.2) (layer "F.Cu") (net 30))
 (segment (start 105.1 122) (end 116.735 110.365) (width 0.2) (layer "F.Cu") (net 30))
 (segment (start 121.579 166) (end 141 166) (width 0.2) (layer "F.Cu") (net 35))
 (segment (start 125.675 155) (end 118.675 148) (width 0.2) (layer "F.Cu") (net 35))
 (segment (start 141 162) (end 134 155) (width 0.2) (layer "F.Cu") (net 35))
 (segment (start 134 155) (end 125.675 155) (width 0.2) (layer "F.Cu") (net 35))
 (segment (start 141 166) (end 141 162) (width 0.2) (layer "F.Cu") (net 35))
 (segment (start 118.675 148) (end 118.675 153) (width 0.2) (layer "F.Cu") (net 35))
 (segment (start 118.18 162.601) (end 121.579 166) (width 0.2) (layer "F.Cu") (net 35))
 (segment (start 108.401 160.651) (end 105.1 157.35) (width 0.2) (layer "F.Cu") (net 33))
 (segment (start 118.18 160.651) (end 108.401 160.651) (width 0.2) (layer "F.Cu") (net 33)))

